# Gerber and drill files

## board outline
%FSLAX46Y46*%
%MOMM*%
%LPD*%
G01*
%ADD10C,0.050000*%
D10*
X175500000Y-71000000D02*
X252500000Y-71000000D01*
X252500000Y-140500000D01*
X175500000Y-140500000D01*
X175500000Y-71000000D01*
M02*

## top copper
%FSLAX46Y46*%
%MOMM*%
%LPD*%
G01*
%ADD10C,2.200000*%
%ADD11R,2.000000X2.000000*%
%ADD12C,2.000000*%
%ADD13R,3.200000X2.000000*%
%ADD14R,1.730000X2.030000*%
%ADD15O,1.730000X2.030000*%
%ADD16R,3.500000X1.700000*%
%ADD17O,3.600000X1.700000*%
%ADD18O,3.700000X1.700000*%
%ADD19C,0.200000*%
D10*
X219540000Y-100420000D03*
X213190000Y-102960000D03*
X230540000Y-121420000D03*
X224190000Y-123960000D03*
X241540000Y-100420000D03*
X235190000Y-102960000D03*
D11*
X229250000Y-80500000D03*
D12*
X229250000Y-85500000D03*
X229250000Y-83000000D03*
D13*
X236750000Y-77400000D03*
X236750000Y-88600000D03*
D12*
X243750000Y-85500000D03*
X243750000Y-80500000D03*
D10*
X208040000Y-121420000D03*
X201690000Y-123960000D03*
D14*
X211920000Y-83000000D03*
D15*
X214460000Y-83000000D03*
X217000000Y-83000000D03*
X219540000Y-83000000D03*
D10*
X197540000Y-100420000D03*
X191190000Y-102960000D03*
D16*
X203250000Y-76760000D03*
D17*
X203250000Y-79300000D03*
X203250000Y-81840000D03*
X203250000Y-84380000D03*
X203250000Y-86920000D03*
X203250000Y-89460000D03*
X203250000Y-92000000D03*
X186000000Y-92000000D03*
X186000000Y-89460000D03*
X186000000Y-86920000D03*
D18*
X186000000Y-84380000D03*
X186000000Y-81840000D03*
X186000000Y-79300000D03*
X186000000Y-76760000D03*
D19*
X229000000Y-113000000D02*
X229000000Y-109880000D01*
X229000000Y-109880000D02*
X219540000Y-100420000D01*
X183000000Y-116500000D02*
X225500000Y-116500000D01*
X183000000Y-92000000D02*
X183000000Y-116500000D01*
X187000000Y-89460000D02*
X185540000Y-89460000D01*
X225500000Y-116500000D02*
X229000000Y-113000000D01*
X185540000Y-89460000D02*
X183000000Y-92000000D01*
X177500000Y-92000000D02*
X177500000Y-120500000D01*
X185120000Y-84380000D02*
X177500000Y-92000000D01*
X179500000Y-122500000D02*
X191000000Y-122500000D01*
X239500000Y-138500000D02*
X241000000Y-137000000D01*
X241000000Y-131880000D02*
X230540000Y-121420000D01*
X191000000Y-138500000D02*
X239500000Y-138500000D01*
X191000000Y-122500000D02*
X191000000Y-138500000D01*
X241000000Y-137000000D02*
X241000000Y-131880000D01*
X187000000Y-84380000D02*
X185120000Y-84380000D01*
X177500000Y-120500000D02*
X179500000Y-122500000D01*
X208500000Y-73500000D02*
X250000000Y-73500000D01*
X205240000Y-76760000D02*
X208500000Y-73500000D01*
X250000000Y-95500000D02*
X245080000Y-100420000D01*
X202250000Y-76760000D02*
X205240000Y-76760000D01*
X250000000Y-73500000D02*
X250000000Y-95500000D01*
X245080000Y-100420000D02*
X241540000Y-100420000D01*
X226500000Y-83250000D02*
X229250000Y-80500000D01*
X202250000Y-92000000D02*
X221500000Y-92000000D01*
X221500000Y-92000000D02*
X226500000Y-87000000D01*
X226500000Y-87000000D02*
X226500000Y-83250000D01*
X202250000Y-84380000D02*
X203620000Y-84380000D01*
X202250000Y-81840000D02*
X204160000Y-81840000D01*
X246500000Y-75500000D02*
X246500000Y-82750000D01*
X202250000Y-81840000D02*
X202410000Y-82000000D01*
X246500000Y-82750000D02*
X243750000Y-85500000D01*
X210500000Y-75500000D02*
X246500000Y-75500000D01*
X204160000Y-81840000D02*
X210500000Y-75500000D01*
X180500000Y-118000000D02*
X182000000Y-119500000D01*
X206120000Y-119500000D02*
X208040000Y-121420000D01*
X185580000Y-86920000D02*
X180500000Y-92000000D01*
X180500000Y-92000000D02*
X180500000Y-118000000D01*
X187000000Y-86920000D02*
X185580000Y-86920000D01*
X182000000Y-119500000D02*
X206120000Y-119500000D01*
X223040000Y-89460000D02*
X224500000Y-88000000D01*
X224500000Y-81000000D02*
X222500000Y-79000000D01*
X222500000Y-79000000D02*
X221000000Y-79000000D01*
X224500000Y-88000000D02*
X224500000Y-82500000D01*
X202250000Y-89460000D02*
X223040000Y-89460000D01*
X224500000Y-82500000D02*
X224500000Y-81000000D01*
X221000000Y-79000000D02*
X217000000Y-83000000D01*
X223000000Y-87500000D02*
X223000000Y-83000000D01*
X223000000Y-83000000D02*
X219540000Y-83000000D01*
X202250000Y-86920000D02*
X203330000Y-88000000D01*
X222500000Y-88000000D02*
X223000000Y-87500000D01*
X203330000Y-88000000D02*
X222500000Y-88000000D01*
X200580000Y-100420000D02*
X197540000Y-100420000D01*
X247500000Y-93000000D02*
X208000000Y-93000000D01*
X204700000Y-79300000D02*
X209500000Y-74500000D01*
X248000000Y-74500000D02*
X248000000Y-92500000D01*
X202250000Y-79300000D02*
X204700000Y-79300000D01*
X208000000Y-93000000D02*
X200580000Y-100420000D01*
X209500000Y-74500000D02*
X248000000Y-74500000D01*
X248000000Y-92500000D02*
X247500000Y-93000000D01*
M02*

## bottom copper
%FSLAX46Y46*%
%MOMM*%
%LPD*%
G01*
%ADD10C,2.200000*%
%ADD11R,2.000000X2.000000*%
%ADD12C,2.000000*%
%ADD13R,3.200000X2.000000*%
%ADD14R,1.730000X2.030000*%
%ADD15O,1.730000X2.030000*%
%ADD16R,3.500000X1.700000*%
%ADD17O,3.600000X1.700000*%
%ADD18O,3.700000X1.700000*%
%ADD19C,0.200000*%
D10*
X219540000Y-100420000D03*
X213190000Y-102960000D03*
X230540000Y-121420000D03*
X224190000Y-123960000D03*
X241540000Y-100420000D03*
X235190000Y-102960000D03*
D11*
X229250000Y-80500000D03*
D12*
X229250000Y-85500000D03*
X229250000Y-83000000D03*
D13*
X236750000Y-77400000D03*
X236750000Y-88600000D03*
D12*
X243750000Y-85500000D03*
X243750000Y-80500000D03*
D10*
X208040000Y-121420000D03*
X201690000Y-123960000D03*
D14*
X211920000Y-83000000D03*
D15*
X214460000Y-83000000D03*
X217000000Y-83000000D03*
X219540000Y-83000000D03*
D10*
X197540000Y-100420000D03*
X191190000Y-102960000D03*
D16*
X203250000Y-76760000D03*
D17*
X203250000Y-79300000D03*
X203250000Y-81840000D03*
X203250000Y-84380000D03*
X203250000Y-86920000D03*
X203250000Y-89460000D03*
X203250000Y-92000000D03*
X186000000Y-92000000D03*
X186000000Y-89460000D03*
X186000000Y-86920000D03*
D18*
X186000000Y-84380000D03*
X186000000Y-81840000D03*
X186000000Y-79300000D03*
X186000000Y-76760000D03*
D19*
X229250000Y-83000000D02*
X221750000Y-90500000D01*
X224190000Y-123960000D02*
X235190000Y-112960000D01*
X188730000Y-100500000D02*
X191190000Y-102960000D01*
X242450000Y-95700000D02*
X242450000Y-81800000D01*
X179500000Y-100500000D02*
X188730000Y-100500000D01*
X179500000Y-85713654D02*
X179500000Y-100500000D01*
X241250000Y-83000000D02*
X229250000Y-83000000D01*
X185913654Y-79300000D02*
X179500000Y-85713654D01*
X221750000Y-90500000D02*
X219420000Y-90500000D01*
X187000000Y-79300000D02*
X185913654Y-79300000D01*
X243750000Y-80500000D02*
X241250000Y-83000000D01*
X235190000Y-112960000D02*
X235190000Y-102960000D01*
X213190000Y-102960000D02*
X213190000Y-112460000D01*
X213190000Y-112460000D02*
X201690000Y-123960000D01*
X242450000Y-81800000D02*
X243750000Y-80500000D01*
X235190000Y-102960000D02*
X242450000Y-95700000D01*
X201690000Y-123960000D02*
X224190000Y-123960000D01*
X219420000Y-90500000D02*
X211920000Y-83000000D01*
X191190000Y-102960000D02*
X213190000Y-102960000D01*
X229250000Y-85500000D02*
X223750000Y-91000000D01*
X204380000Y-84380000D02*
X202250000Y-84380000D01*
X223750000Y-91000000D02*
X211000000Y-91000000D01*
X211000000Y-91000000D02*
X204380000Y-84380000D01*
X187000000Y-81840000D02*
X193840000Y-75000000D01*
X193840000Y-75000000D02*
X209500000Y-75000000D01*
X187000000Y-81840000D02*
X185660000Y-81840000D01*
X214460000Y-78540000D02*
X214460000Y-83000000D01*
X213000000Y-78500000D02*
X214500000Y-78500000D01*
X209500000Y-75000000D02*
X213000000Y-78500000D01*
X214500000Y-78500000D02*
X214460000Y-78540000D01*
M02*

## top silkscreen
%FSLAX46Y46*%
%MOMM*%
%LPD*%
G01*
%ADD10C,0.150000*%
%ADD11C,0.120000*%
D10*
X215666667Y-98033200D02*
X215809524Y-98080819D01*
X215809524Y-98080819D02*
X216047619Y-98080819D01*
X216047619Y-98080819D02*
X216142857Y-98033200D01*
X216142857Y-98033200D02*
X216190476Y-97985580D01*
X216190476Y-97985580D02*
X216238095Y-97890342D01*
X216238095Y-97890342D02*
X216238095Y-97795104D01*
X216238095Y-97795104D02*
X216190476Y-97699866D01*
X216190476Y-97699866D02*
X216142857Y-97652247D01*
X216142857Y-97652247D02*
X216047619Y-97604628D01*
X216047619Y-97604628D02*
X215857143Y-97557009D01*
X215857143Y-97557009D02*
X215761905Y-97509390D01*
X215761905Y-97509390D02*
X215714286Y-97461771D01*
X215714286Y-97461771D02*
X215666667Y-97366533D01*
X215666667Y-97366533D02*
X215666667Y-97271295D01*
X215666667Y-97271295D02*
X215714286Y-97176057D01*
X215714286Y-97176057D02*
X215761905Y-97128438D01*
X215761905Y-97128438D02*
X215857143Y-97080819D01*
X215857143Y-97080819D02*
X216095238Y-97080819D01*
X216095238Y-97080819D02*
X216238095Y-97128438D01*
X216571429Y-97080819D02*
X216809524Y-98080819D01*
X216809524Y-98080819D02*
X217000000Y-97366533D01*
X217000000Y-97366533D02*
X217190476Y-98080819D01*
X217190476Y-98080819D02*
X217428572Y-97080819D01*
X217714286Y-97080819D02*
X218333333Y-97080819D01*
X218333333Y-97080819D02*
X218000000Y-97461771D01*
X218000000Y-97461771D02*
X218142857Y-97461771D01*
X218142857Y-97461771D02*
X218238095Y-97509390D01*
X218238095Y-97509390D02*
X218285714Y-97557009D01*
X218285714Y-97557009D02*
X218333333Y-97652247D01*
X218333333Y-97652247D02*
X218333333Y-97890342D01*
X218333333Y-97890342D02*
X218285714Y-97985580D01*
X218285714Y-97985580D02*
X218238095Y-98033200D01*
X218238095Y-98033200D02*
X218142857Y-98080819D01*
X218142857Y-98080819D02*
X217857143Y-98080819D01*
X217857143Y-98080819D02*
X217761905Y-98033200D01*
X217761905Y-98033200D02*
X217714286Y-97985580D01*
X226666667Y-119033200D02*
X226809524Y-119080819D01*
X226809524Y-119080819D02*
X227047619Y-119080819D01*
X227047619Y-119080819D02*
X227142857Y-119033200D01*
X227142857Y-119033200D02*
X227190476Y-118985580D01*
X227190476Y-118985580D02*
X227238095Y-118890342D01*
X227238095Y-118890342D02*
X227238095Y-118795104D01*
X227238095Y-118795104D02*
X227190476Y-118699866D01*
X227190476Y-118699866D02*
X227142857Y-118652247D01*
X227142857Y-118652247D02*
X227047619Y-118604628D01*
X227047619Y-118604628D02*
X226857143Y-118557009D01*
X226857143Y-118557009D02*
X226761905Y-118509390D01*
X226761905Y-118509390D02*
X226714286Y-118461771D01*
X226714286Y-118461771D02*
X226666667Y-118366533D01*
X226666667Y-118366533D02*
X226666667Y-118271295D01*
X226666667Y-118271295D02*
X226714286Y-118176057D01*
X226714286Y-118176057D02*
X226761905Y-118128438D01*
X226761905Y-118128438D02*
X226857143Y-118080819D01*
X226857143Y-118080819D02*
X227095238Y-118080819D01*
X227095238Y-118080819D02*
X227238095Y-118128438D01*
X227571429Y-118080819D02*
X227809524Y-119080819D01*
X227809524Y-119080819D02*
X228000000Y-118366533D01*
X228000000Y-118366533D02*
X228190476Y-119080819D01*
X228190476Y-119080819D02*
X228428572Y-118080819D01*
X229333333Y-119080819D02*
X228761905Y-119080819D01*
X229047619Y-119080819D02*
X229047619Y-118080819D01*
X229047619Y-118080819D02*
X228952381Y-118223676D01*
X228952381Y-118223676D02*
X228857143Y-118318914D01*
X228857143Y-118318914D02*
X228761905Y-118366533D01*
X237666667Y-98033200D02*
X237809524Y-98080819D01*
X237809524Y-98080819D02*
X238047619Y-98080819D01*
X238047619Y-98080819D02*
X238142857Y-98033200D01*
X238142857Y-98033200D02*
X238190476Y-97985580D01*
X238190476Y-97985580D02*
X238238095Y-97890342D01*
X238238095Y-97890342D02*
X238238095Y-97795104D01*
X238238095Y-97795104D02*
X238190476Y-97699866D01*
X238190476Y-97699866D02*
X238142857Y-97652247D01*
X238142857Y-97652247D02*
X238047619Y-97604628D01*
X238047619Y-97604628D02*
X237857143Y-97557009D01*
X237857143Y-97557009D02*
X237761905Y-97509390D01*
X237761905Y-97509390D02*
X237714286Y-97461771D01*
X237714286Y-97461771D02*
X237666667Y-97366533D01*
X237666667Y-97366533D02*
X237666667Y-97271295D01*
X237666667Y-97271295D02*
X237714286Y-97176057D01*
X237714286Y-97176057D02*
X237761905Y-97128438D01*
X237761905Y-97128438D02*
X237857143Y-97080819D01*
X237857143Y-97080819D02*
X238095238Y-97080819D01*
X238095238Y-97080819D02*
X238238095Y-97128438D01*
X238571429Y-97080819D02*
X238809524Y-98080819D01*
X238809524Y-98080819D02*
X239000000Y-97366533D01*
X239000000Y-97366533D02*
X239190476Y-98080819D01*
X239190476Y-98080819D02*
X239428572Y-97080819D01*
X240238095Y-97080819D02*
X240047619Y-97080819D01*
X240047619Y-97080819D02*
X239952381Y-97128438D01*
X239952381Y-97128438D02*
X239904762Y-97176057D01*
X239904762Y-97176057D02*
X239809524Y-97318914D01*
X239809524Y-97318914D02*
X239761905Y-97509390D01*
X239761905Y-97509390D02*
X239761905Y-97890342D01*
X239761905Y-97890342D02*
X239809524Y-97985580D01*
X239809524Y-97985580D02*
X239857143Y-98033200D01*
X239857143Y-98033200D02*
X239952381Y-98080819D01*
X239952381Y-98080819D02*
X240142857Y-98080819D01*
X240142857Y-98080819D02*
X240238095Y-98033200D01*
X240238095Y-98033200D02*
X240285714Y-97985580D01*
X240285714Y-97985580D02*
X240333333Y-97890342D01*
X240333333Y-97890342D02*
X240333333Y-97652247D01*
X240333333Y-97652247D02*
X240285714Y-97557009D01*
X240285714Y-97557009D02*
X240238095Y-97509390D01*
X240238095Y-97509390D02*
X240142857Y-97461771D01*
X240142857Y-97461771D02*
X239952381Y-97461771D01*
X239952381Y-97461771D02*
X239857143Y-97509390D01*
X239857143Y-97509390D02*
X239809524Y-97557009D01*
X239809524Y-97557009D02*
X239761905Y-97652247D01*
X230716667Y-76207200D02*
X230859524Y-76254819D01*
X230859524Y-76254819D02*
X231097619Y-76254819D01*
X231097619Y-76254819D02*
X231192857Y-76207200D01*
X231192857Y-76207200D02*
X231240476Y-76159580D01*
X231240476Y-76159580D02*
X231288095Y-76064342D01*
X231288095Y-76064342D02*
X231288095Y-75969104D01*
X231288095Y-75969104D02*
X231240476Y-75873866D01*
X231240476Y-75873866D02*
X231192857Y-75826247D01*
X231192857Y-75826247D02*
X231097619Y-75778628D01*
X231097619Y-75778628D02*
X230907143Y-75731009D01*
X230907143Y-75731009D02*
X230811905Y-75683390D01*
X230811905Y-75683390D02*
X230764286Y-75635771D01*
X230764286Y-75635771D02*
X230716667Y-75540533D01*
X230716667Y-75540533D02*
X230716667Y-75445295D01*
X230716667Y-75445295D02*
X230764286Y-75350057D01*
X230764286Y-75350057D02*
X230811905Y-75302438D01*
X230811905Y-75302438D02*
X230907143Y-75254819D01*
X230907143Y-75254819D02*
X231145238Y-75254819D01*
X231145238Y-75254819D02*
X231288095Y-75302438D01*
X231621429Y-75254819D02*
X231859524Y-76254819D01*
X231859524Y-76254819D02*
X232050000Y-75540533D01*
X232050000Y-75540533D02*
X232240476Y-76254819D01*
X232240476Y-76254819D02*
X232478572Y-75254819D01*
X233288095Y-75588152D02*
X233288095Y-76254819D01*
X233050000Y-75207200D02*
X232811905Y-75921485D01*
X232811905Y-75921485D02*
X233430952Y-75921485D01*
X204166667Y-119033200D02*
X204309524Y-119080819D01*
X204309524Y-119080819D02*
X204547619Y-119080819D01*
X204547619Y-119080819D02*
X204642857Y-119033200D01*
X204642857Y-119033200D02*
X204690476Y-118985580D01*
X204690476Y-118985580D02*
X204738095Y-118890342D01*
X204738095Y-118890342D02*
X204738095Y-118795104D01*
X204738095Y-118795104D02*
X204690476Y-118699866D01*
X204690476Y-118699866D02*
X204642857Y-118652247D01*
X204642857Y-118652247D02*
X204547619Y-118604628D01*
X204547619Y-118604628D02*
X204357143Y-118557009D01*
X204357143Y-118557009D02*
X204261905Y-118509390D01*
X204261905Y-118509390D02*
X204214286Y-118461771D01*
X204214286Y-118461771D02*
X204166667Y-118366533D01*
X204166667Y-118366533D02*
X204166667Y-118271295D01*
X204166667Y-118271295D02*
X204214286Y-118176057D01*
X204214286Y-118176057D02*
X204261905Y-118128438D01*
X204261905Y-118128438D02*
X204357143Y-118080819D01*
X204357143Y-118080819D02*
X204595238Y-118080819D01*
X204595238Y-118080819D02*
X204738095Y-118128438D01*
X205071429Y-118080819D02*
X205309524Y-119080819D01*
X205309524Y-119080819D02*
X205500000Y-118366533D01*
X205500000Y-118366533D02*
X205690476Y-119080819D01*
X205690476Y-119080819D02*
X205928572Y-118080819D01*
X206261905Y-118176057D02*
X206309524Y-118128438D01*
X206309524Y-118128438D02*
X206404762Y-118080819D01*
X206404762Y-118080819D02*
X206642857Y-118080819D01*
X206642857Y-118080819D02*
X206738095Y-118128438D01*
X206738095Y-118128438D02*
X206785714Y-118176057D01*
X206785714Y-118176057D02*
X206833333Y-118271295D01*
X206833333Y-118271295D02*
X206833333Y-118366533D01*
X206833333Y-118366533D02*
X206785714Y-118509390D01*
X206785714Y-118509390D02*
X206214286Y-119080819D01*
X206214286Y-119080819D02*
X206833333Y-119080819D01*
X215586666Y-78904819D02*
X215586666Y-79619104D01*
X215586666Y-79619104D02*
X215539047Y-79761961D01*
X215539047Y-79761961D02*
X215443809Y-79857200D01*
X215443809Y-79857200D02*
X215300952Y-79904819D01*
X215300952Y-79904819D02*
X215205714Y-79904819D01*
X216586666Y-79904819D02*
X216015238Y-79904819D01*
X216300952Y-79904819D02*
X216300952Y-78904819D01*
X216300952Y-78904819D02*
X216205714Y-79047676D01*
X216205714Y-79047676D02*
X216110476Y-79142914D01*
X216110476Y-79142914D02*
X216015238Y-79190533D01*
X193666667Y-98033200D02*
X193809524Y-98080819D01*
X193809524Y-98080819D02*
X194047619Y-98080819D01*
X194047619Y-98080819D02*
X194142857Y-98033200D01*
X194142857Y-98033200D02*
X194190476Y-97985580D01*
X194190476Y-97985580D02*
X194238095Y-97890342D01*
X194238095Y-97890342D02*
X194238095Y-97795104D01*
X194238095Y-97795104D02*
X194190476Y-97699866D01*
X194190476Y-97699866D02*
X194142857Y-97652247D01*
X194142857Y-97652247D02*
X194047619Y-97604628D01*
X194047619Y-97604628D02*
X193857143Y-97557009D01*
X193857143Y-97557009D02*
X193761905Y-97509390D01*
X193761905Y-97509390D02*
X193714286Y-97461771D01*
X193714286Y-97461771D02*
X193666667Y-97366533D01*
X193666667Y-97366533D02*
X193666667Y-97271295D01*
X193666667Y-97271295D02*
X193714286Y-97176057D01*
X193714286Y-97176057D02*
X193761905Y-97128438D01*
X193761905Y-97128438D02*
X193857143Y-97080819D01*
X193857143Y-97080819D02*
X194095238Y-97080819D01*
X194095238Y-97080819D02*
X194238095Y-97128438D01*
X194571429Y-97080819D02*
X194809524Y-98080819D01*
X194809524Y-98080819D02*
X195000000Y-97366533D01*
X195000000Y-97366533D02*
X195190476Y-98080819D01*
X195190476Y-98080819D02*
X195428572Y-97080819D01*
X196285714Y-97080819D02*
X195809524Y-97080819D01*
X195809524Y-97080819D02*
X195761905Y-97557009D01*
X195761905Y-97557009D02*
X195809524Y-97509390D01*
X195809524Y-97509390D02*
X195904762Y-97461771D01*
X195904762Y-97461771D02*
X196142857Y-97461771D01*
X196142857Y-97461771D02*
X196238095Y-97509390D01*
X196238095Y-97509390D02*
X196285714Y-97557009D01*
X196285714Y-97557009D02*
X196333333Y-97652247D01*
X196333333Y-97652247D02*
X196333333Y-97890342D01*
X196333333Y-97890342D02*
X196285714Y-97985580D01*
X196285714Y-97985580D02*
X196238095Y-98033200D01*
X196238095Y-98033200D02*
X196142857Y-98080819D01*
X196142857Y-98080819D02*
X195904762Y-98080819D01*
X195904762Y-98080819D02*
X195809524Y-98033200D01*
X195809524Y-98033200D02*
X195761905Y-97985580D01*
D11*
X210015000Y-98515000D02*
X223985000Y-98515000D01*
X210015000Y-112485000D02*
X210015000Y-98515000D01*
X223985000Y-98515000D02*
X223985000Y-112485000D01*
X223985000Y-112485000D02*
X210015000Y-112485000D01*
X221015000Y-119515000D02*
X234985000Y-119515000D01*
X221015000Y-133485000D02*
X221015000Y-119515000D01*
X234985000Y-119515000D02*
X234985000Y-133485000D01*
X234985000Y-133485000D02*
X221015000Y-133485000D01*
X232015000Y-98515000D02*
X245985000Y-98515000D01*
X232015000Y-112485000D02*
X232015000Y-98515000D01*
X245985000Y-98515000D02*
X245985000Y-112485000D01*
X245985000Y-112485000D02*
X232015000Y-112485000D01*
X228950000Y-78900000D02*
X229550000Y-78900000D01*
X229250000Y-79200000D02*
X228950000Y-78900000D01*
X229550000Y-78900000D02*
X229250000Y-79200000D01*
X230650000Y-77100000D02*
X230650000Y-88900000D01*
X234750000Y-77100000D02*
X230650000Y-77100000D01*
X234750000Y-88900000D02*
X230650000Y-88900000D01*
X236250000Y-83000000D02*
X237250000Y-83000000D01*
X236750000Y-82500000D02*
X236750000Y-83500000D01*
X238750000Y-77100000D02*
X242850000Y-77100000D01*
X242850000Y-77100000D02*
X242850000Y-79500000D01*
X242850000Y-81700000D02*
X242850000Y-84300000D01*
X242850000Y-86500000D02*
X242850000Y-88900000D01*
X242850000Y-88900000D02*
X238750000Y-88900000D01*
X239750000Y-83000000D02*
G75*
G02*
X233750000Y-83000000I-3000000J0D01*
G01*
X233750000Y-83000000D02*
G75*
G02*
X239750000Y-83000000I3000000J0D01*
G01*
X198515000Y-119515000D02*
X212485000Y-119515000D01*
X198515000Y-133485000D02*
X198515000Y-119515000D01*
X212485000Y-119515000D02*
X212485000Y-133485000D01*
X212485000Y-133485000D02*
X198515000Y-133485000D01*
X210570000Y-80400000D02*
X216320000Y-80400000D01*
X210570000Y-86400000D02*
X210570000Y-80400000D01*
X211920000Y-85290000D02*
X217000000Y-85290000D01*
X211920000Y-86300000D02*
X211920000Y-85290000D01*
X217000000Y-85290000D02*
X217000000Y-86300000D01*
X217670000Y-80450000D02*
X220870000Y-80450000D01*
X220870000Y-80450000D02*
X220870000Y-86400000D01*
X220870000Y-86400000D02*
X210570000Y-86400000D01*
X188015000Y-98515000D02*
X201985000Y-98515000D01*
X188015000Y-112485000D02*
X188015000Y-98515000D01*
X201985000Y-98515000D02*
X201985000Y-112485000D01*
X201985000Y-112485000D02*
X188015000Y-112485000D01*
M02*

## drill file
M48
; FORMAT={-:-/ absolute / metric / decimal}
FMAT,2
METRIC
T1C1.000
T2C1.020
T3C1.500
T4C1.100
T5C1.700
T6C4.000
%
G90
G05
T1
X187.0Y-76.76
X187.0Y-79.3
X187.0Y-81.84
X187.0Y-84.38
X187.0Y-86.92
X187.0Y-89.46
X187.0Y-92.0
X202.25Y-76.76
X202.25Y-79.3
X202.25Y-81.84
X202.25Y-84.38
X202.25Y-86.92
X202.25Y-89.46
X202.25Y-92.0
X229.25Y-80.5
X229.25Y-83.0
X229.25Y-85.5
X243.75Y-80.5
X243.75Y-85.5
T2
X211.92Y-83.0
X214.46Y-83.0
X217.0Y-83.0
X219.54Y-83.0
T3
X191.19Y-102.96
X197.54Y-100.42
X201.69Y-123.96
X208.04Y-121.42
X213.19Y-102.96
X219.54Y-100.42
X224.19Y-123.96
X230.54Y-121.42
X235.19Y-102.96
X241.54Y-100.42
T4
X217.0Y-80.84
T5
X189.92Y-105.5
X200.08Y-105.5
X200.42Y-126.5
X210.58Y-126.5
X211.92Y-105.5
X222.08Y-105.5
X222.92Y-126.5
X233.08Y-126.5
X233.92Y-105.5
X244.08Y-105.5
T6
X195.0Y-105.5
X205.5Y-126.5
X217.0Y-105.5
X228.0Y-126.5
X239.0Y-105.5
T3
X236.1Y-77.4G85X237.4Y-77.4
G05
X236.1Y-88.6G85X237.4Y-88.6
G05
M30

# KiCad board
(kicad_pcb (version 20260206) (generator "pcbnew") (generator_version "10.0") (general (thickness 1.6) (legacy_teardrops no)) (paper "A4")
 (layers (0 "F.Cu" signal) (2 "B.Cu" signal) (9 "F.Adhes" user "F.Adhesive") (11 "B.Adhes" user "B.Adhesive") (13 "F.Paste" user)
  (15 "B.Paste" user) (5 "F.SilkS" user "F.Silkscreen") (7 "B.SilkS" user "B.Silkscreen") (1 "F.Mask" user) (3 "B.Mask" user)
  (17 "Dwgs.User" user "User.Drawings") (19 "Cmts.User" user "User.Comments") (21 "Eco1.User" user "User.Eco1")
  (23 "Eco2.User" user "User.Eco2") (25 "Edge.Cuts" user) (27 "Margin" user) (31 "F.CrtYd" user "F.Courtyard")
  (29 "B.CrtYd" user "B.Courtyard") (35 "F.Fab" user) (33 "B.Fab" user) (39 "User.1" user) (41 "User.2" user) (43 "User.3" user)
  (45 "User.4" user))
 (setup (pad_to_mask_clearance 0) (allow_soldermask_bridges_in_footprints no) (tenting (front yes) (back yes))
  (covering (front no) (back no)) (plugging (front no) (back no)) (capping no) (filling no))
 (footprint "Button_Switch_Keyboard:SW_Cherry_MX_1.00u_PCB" (layer "F.Cu") (at 219.54 100.42)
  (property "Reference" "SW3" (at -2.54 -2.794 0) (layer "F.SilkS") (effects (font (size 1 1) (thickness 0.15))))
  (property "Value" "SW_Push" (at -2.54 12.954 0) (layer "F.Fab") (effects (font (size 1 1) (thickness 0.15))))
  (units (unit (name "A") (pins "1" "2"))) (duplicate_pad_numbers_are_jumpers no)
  (fp_line (start -9.525 -1.905) (end 4.445 -1.905) (stroke (width 0.12) (type solid)) (layer "F.SilkS"))
  (fp_line (start -9.525 12.065) (end -9.525 -1.905) (stroke (width 0.12) (type solid)) (layer "F.SilkS"))
  (fp_line (start 4.445 -1.905) (end 4.445 12.065) (stroke (width 0.12) (type solid)) (layer "F.SilkS"))
  (fp_line (start 4.445 12.065) (end -9.525 12.065) (stroke (width 0.12) (type solid)) (layer "F.SilkS"))
  (pad "" np_thru_hole circle (at -7.62 5.08) (size 1.7 1.7) (drill 1.7) (layers "*.Cu" "*.Mask"))
  (pad "" np_thru_hole circle (at -2.54 5.08) (size 4 4) (drill 4) (layers "*.Cu" "*.Mask"))
  (pad "" np_thru_hole circle (at 2.54 5.08) (size 1.7 1.7) (drill 1.7) (layers "*.Cu" "*.Mask"))
  (pad "1" thru_hole circle (at 0 0) (size 2.2 2.2) (drill 1.5) (layers "*.Cu" "*.Mask") (remove_unused_layers no)
   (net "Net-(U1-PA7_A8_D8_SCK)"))
  (pad "2" thru_hole circle (at -6.35 2.54) (size 2.2 2.2) (drill 1.5) (layers "*.Cu" "*.Mask") (remove_unused_layers no) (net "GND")))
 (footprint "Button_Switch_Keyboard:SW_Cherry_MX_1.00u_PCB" (layer "F.Cu") (at 230.54 121.42)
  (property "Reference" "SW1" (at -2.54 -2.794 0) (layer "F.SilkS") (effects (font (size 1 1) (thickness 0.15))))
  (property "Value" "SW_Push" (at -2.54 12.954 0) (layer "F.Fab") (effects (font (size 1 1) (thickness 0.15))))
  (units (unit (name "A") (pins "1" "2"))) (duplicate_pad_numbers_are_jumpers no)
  (fp_line (start -9.525 -1.905) (end 4.445 -1.905) (stroke (width 0.12) (type solid)) (layer "F.SilkS"))
  (fp_line (start -9.525 12.065) (end -9.525 -1.905) (stroke (width 0.12) (type solid)) (layer "F.SilkS"))
  (fp_line (start 4.445 -1.905) (end 4.445 12.065) (stroke (width 0.12) (type solid)) (layer "F.SilkS"))
  (fp_line (start 4.445 12.065) (end -9.525 12.065) (stroke (width 0.12) (type solid)) (layer "F.SilkS"))
  (pad "" np_thru_hole circle (at -7.62 5.08) (size 1.7 1.7) (drill 1.7) (layers "*.Cu" "*.Mask"))
  (pad "" np_thru_hole circle (at -2.54 5.08) (size 4 4) (drill 4) (layers "*.Cu" "*.Mask"))
  (pad "" np_thru_hole circle (at 2.54 5.08) (size 1.7 1.7) (drill 1.7) (layers "*.Cu" "*.Mask"))
  (pad "1" thru_hole circle (at 0 0) (size 2.2 2.2) (drill 1.5) (layers "*.Cu" "*.Mask") (remove_unused_layers no)
   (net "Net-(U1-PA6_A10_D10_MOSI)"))
  (pad "2" thru_hole circle (at -6.35 2.54) (size 2.2 2.2) (drill 1.5) (layers "*.Cu" "*.Mask") (remove_unused_layers no) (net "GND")))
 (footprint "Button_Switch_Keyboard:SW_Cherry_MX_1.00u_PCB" (layer "F.Cu") (at 241.54 100.42)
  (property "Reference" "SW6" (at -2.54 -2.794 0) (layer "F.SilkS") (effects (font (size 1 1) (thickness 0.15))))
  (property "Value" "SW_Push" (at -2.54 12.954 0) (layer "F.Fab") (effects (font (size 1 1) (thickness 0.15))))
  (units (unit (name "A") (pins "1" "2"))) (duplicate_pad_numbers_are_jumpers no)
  (fp_line (start -9.525 -1.905) (end 4.445 -1.905) (stroke (width 0.12) (type solid)) (layer "F.SilkS"))
  (fp_line (start -9.525 12.065) (end -9.525 -1.905) (stroke (width 0.12) (type solid)) (layer "F.SilkS"))
  (fp_line (start 4.445 -1.905) (end 4.445 12.065) (stroke (width 0.12) (type solid)) (layer "F.SilkS"))
  (fp_line (start 4.445 12.065) (end -9.525 12.065) (stroke (width 0.12) (type solid)) (layer "F.SilkS"))
  (pad "" np_thru_hole circle (at -7.62 5.08) (size 1.7 1.7) (drill 1.7) (layers "*.Cu" "*.Mask"))
  (pad "" np_thru_hole circle (at -2.54 5.08) (size 4 4) (drill 4) (layers "*.Cu" "*.Mask"))
  (pad "" np_thru_hole circle (at 2.54 5.08) (size 1.7 1.7) (drill 1.7) (layers "*.Cu" "*.Mask"))
  (pad "1" thru_hole circle (at 0 0) (size 2.2 2.2) (drill 1.5) (layers "*.Cu" "*.Mask") (remove_unused_layers no)
   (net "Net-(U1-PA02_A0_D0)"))
  (pad "2" thru_hole circle (at -6.35 2.54) (size 2.2 2.2) (drill 1.5) (layers "*.Cu" "*.Mask") (remove_unused_layers no) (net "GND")))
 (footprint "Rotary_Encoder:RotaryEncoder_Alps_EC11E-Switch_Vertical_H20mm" (layer "F.Cu") (at 229.25 80.5)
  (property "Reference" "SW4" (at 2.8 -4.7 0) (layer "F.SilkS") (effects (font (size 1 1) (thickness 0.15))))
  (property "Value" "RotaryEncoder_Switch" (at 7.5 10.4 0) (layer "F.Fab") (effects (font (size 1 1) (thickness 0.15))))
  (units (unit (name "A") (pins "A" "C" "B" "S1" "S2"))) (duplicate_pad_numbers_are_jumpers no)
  (fp_line (start -0.3 -1.6) (end 0.3 -1.6) (stroke (width 0.12) (type solid)) (layer "F.SilkS"))
  (fp_line (start 0 -1.3) (end -0.3 -1.6) (stroke (width 0.12) (type solid)) (layer "F.SilkS"))
  (fp_line (start 0.3 -1.6) (end 0 -1.3) (stroke (width 0.12) (type solid)) (layer "F.SilkS"))
  (fp_line (start 1.4 -3.4) (end 1.4 8.4) (stroke (width 0.12) (type solid)) (layer "F.SilkS"))
  (fp_line (start 5.5 -3.4) (end 1.4 -3.4) (stroke (width 0.12) (type solid)) (layer "F.SilkS"))
  (fp_line (start 5.5 8.4) (end 1.4 8.4) (stroke (width 0.12) (type solid)) (layer "F.SilkS"))
  (fp_line (start 7 2.5) (end 8 2.5) (stroke (width 0.12) (type solid)) (layer "F.SilkS"))
  (fp_line (start 7.5 2) (end 7.5 3) (stroke (width 0.12) (type solid)) (layer "F.SilkS"))
  (fp_line (start 9.5 -3.4) (end 13.6 -3.4) (stroke (width 0.12) (type solid)) (layer "F.SilkS"))
  (fp_line (start 13.6 -3.4) (end 13.6 -1) (stroke (width 0.12) (type solid)) (layer "F.SilkS"))
  (fp_line (start 13.6 1.2) (end 13.6 3.8) (stroke (width 0.12) (type solid)) (layer "F.SilkS"))
  (fp_line (start 13.6 6) (end 13.6 8.4) (stroke (width 0.12) (type solid)) (layer "F.SilkS"))
  (fp_line (start 13.6 8.4) (end 9.5 8.4) (stroke (width 0.12) (type solid)) (layer "F.SilkS"))
  (fp_circle (center 7.5 2.5) (end 10.5 2.5) (stroke (width 0.12) (type solid)) (fill no) (layer "F.SilkS"))
  (pad "A" thru_hole rect (at 0 0) (size 2 2) (drill 1) (layers "*.Cu" "*.Mask") (remove_unused_layers no) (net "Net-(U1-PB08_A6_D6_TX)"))
  (pad "B" thru_hole circle (at 0 5) (size 2 2) (drill 1) (layers "*.Cu" "*.Mask") (remove_unused_layers no) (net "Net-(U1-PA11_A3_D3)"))
  (pad "C" thru_hole circle (at 0 2.5) (size 2 2) (drill 1) (layers "*.Cu" "*.Mask") (remove_unused_layers no) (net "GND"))
  (pad "MP" thru_hole rect (at 7.5 -3.1) (size 3.2 2) (drill oval 2.8 1.5) (layers "*.Cu" "*.Mask") (remove_unused_layers no))
  (pad "MP" thru_hole rect (at 7.5 8.1) (size 3.2 2) (drill oval 2.8 1.5) (layers "*.Cu" "*.Mask") (remove_unused_layers no))
  (pad "S1" thru_hole circle (at 14.5 5) (size 2 2) (drill 1) (layers "*.Cu" "*.Mask") (remove_unused_layers no) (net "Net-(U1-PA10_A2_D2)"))
  (pad "S2" thru_hole circle (at 14.5 0) (size 2 2) (drill 1) (layers "*.Cu" "*.Mask") (remove_unused_layers no) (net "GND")))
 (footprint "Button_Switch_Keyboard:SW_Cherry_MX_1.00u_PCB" (layer "F.Cu") (at 208.04 121.42)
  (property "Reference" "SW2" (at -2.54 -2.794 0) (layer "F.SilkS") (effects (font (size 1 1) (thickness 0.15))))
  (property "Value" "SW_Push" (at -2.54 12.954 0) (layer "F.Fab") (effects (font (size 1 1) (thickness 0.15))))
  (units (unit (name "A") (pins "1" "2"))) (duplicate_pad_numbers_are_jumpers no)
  (fp_line (start -9.525 -1.905) (end 4.445 -1.905) (stroke (width 0.12) (type solid)) (layer "F.SilkS"))
  (fp_line (start -9.525 12.065) (end -9.525 -1.905) (stroke (width 0.12) (type solid)) (layer "F.SilkS"))
  (fp_line (start 4.445 -1.905) (end 4.445 12.065) (stroke (width 0.12) (type solid)) (layer "F.SilkS"))
  (fp_line (start 4.445 12.065) (end -9.525 12.065) (stroke (width 0.12) (type solid)) (layer "F.SilkS"))
  (pad "" np_thru_hole circle (at -7.62 5.08) (size 1.7 1.7) (drill 1.7) (layers "*.Cu" "*.Mask"))
  (pad "" np_thru_hole circle (at -2.54 5.08) (size 4 4) (drill 4) (layers "*.Cu" "*.Mask"))
  (pad "" np_thru_hole circle (at 2.54 5.08) (size 1.7 1.7) (drill 1.7) (layers "*.Cu" "*.Mask"))
  (pad "1" thru_hole circle (at 0 0) (size 2.2 2.2) (drill 1.5) (layers "*.Cu" "*.Mask") (remove_unused_layers no)
   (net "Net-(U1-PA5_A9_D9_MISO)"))
  (pad "2" thru_hole circle (at -6.35 2.54) (size 2.2 2.2) (drill 1.5) (layers "*.Cu" "*.Mask") (remove_unused_layers no) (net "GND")))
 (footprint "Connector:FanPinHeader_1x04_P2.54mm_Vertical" (layer "F.Cu") (at 211.92 83)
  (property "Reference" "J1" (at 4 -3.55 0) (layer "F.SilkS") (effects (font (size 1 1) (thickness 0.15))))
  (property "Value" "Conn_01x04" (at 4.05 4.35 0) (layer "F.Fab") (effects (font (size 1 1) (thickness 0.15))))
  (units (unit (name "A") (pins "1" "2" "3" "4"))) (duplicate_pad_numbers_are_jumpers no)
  (fp_line (start -1.35 -2.6) (end 4.4 -2.6) (stroke (width 0.12) (type solid)) (layer "F.SilkS"))
  (fp_line (start -1.35 3.4) (end -1.35 -2.6) (stroke (width 0.12) (type solid)) (layer "F.SilkS"))
  (fp_line (start 0 2.29) (end 5.08 2.29) (stroke (width 0.12) (type solid)) (layer "F.SilkS"))
  (fp_line (start 0 3.3) (end 0 2.29) (stroke (width 0.12) (type solid)) (layer "F.SilkS"))
  (fp_line (start 5.08 2.29) (end 5.08 3.3) (stroke (width 0.12) (type solid)) (layer "F.SilkS"))
  (fp_line (start 5.75 -2.55) (end 8.95 -2.55) (stroke (width 0.12) (type solid)) (layer "F.SilkS"))
  (fp_line (start 8.95 -2.55) (end 8.95 3.4) (stroke (width 0.12) (type solid)) (layer "F.SilkS"))
  (fp_line (start 8.95 3.4) (end -1.35 3.4) (stroke (width 0.12) (type solid)) (layer "F.SilkS"))
  (pad "" np_thru_hole circle (at 5.08 -2.16 90) (size 1.1 1.1) (drill 1.1) (layers "*.Cu" "*.Mask"))
  (pad "1" thru_hole rect (at 0 0 90) (size 2.03 1.73) (drill 1.02) (layers "*.Cu" "*.Mask") (remove_unused_layers no) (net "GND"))
  (pad "2" thru_hole oval (at 2.54 0 90) (size 2.03 1.73) (drill 1.02) (layers "*.Cu" "*.Mask") (remove_unused_layers no) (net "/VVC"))
  (pad "3" thru_hole oval (at 5.08 0 90) (size 2.03 1.73) (drill 1.02) (layers "*.Cu" "*.Mask") (remove_unused_layers no) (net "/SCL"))
  (pad "4" thru_hole oval (at 7.62 0 90) (size 2.03 1.73) (drill 1.02) (layers "*.Cu" "*.Mask") (remove_unused_layers no) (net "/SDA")))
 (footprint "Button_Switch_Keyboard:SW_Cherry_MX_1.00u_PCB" (layer "F.Cu") (at 197.54 100.42)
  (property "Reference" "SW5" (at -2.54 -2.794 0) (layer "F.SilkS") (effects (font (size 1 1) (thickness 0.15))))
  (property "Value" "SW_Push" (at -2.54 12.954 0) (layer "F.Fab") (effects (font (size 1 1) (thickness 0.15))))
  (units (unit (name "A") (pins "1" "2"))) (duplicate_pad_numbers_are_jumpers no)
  (fp_line (start -9.525 -1.905) (end 4.445 -1.905) (stroke (width 0.12) (type solid)) (layer "F.SilkS"))
  (fp_line (start -9.525 12.065) (end -9.525 -1.905) (stroke (width 0.12) (type solid)) (layer "F.SilkS"))
  (fp_line (start 4.445 -1.905) (end 4.445 12.065) (stroke (width 0.12) (type solid)) (layer "F.SilkS"))
  (fp_line (start 4.445 12.065) (end -9.525 12.065) (stroke (width 0.12) (type solid)) (layer "F.SilkS"))
  (pad "" np_thru_hole circle (at -7.62 5.08) (size 1.7 1.7) (drill 1.7) (layers "*.Cu" "*.Mask"))
  (pad "" np_thru_hole circle (at -2.54 5.08) (size 4 4) (drill 4) (layers "*.Cu" "*.Mask"))
  (pad "" np_thru_hole circle (at 2.54 5.08) (size 1.7 1.7) (drill 1.7) (layers "*.Cu" "*.Mask"))
  (pad "1" thru_hole circle (at 0 0) (size 2.2 2.2) (drill 1.5) (layers "*.Cu" "*.Mask") (remove_unused_layers no)
   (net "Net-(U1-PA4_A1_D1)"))
  (pad "2" thru_hole circle (at -6.35 2.54) (size 2.2 2.2) (drill 1.5) (layers "*.Cu" "*.Mask") (remove_unused_layers no) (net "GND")))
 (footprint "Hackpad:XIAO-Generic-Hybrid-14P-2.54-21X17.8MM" (layer "B.Cu") (at 194.625 84.38 180)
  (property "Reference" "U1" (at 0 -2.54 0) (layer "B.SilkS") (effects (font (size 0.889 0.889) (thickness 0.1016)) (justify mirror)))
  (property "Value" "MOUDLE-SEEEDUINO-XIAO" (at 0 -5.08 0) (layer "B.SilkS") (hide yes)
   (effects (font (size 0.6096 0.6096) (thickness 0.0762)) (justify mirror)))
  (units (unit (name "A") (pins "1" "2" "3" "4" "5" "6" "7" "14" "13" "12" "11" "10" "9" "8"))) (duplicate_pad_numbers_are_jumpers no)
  (pad "1" thru_hole rect (at -7.625 7.62 180) (size 3.5 1.7) (drill 1 (offset -1 0)) (layers "*.Cu" "*.Mask") (remove_unused_layers no)
   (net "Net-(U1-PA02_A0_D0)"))
  (pad "2" thru_hole oval (at -7.625 5.08 180) (size 3.6 1.7) (drill 1 (offset -1 0)) (layers "*.Cu" "*.Mask") (remove_unused_layers no)
   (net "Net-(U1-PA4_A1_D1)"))
  (pad "3" thru_hole oval (at -7.625 2.54 180) (size 3.6 1.7) (drill 1 (offset -1 0)) (layers "*.Cu" "*.Mask") (remove_unused_layers no)
   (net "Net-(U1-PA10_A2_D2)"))
  (pad "4" thru_hole oval (at -7.625 0 180) (size 3.6 1.7) (drill 1 (offset -1 0)) (layers "*.Cu" "*.Mask") (remove_unused_layers no)
   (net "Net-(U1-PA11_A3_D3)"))
  (pad "5" thru_hole oval (at -7.625 -2.54 180) (size 3.6 1.7) (drill 1 (offset -1 0)) (layers "*.Cu" "*.Mask") (remove_unused_layers no)
   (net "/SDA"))
  (pad "6" thru_hole oval (at -7.625 -5.08) (size 3.6 1.7) (drill 1 (offset 1 0)) (layers "*.Cu" "*.Mask") (remove_unused_layers no)
   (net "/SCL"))
  (pad "7" thru_hole oval (at -7.625 -7.62 180) (size 3.6 1.7) (drill 1 (offset -1 0)) (layers "*.Cu" "*.Mask") (remove_unused_layers no)
   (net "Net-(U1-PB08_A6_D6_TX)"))
  (pad "8" thru_hole oval (at 7.625 -7.62 180) (size 3.6 1.7) (drill 1 (offset 1 0)) (layers "*.Cu" "*.Mask") (remove_unused_layers no)
   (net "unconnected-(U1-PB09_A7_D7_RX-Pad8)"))
  (pad "9" thru_hole oval (at 7.625 -5.08 180) (size 3.6 1.7) (drill 1 (offset 1 0)) (layers "*.Cu" "*.Mask") (remove_unused_layers no)
   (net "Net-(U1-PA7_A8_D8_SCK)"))
  (pad "10" thru_hole oval (at 7.625 -2.54 180) (size 3.6 1.7) (drill 1 (offset 1 0)) (layers "*.Cu" "*.Mask") (remove_unused_layers no)
   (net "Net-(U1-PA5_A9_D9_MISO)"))
  (pad "11" thru_hole oval (at 7.625 0 180) (size 3.7 1.7) (drill 1 (offset 1 0)) (layers "*.Cu" "*.Mask") (remove_unused_layers no)
   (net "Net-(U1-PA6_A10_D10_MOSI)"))
  (pad "12" thru_hole oval (at 7.625 2.54 180) (size 3.7 1.7) (drill 1 (offset 1 0)) (layers "*.Cu" "*.Mask") (remove_unused_layers no)
   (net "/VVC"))
  (pad "13" thru_hole oval (at 7.625 5.08 180) (size 3.7 1.7) (drill 1 (offset 1 0)) (layers "*.Cu" "*.Mask") (remove_unused_layers no)
   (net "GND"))
  (pad "14" thru_hole oval (at 7.625 7.62 180) (size 3.7 1.7) (drill 1 (offset 1 0)) (layers "*.Cu" "*.Mask") (remove_unused_layers no)
   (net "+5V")))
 (gr_rect (start 175.5 71) (end 252.5 140.5) (stroke (width 0.05) (type default)) (fill no) (layer "Edge.Cuts"))
 (segment (start 229 113) (end 229 109.88) (width 0.2) (layer "F.Cu") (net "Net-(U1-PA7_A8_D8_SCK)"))
 (segment (start 229 109.88) (end 219.54 100.42) (width 0.2) (layer "F.Cu") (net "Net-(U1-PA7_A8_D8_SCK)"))
 (segment (start 183 116.5) (end 225.5 116.5) (width 0.2) (layer "F.Cu") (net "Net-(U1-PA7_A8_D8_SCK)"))
 (segment (start 183 92) (end 183 116.5) (width 0.2) (layer "F.Cu") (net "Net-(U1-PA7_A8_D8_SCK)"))
 (segment (start 187 89.46) (end 185.54 89.46) (width 0.2) (layer "F.Cu") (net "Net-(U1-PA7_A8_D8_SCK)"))
 (segment (start 225.5 116.5) (end 229 113) (width 0.2) (layer "F.Cu") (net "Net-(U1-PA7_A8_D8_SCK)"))
 (segment (start 185.54 89.46) (end 183 92) (width 0.2) (layer "F.Cu") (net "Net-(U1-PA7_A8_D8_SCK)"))
 (segment (start 229.25 83) (end 221.75 90.5) (width 0.2) (layer "B.Cu") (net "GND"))
 (segment (start 224.19 123.96) (end 235.19 112.96) (width 0.2) (layer "B.Cu") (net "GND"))
 (segment (start 188.73 100.5) (end 191.19 102.96) (width 0.2) (layer "B.Cu") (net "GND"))
 (segment (start 242.45 95.7) (end 242.45 81.8) (width 0.2) (layer "B.Cu") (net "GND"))
 (segment (start 179.5 100.5) (end 188.73 100.5) (width 0.2) (layer "B.Cu") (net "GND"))
 (segment (start 179.5 85.713654) (end 179.5 100.5) (width 0.2) (layer "B.Cu") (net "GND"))
 (segment (start 241.25 83) (end 229.25 83) (width 0.2) (layer "B.Cu") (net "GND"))
 (segment (start 185.913654 79.3) (end 179.5 85.713654) (width 0.2) (layer "B.Cu") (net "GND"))
 (segment (start 221.75 90.5) (end 219.42 90.5) (width 0.2) (layer "B.Cu") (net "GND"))
 (segment (start 187 79.3) (end 185.913654 79.3) (width 0.2) (layer "B.Cu") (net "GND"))
 (segment (start 243.75 80.5) (end 241.25 83) (width 0.2) (layer "B.Cu") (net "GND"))
 (segment (start 235.19 112.96) (end 235.19 102.96) (width 0.2) (layer "B.Cu") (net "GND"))
 (segment (start 213.19 102.96) (end 213.19 112.46) (width 0.2) (layer "B.Cu") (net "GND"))
 (segment (start 213.19 112.46) (end 201.69 123.96) (width 0.2) (layer "B.Cu") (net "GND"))
 (segment (start 242.45 81.8) (end 243.75 80.5) (width 0.2) (layer "B.Cu") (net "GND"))
 (segment (start 235.19 102.96) (end 242.45 95.7) (width 0.2) (layer "B.Cu") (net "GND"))
 (segment (start 201.69 123.96) (end 224.19 123.96) (width 0.2) (layer "B.Cu") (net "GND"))
 (segment (start 219.42 90.5) (end 211.92 83) (width 0.2) (layer "B.Cu") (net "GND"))
 (segment (start 191.19 102.96) (end 213.19 102.96) (width 0.2) (layer "B.Cu") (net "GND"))
 (segment (start 177.5 92) (end 177.5 120.5) (width 0.2) (layer "F.Cu") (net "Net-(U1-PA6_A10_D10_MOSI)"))
 (segment (start 185.12 84.38) (end 177.5 92) (width 0.2) (layer "F.Cu") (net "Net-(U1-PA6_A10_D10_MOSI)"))
 (segment (start 179.5 122.5) (end 191 122.5) (width 0.2) (layer "F.Cu") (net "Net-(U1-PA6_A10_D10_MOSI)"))
 (segment (start 239.5 138.5) (end 241 137) (width 0.2) (layer "F.Cu") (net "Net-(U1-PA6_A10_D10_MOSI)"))
 (segment (start 241 131.88) (end 230.54 121.42) (width 0.2) (layer "F.Cu") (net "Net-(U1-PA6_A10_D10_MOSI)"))
 (segment (start 191 138.5) (end 239.5 138.5) (width 0.2) (layer "F.Cu") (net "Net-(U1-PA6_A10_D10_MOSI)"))
 (segment (start 191 122.5) (end 191 138.5) (width 0.2) (layer "F.Cu") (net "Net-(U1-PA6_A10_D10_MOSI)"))
 (segment (start 241 137) (end 241 131.88) (width 0.2) (layer "F.Cu") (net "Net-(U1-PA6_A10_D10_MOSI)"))
 (segment (start 187 84.38) (end 185.12 84.38) (width 0.2) (layer "F.Cu") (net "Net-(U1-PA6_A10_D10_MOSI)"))
 (segment (start 177.5 120.5) (end 179.5 122.5) (width 0.2) (layer "F.Cu") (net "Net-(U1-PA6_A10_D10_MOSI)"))
 (segment (start 208.5 73.5) (end 250 73.5) (width 0.2) (layer "F.Cu") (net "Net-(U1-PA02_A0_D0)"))
 (segment (start 205.24 76.76) (end 208.5 73.5) (width 0.2) (layer "F.Cu") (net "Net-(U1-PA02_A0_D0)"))
 (segment (start 250 95.5) (end 245.08 100.42) (width 0.2) (layer "F.Cu") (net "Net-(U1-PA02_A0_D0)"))
 (segment (start 202.25 76.76) (end 205.24 76.76) (width 0.2) (layer "F.Cu") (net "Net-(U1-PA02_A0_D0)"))
 (segment (start 250 73.5) (end 250 95.5) (width 0.2) (layer "F.Cu") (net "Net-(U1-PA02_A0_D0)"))
 (segment (start 245.08 100.42) (end 241.54 100.42) (width 0.2) (layer "F.Cu") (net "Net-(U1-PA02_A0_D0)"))
 (segment (start 226.5 83.25) (end 229.25 80.5) (width 0.2) (layer "F.Cu") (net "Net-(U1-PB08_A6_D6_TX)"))
 (segment (start 202.25 92) (end 221.5 92) (width 0.2) (layer "F.Cu") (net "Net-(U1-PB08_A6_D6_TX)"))
 (segment (start 221.5 92) (end 226.5 87) (width 0.2) (layer "F.Cu") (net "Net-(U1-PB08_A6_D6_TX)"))
 (segment (start 226.5 87) (end 226.5 83.25) (width 0.2) (layer "F.Cu") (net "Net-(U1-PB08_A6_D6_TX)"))
 (segment (start 202.25 84.38) (end 203.62 84.38) (width 0.2) (layer "F.Cu") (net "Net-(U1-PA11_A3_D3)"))
 (segment (start 229.25 85.5) (end 223.75 91) (width 0.2) (layer "B.Cu") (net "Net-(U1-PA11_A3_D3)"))
 (segment (start 204.38 84.38) (end 202.25 84.38) (width 0.2) (layer "B.Cu") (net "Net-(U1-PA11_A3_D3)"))
 (segment (start 223.75 91) (end 211 91) (width 0.2) (layer "B.Cu") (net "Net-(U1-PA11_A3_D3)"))
 (segment (start 211 91) (end 204.38 84.38) (width 0.2) (layer "B.Cu") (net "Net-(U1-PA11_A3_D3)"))
 (segment (start 202.25 81.84) (end 204.16 81.84) (width 0.2) (layer "F.Cu") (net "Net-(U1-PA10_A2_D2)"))
 (segment (start 246.5 75.5) (end 246.5 82.75) (width 0.2) (layer "F.Cu") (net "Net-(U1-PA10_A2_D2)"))
 (segment (start 202.25 81.84) (end 202.41 82) (width 0.2) (layer "F.Cu") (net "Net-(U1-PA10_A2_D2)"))
 (segment (start 246.5 82.75) (end 243.75 85.5) (width 0.2) (layer "F.Cu") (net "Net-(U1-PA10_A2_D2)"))
 (segment (start 210.5 75.5) (end 246.5 75.5) (width 0.2) (layer "F.Cu") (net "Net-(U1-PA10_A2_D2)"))
 (segment (start 204.16 81.84) (end 210.5 75.5) (width 0.2) (layer "F.Cu") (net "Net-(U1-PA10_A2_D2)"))
 (segment (start 180.5 118) (end 182 119.5) (width 0.2) (layer "F.Cu") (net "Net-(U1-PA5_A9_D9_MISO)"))
 (segment (start 206.12 119.5) (end 208.04 121.42) (width 0.2) (layer "F.Cu") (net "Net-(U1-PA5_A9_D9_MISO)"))
 (segment (start 185.58 86.92) (end 180.5 92) (width 0.2) (layer "F.Cu") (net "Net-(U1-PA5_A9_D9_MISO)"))
 (segment (start 180.5 92) (end 180.5 118) (width 0.2) (layer "F.Cu") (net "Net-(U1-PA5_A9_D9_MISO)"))
 (segment (start 187 86.92) (end 185.58 86.92) (width 0.2) (layer "F.Cu") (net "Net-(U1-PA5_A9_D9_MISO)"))
 (segment (start 182 119.5) (end 206.12 119.5) (width 0.2) (layer "F.Cu") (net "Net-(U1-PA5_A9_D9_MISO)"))
 (segment (start 187 81.84) (end 193.84 75) (width 0.2) (layer "B.Cu") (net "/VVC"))
 (segment (start 193.84 75) (end 209.5 75) (width 0.2) (layer "B.Cu") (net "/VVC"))
 (segment (start 187 81.84) (end 185.66 81.84) (width 0.2) (layer "B.Cu") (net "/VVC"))
 (segment (start 214.46 78.54) (end 214.46 83) (width 0.2) (layer "B.Cu") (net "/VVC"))
 (segment (start 213 78.5) (end 214.5 78.5) (width 0.2) (layer "B.Cu") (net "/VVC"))
 (segment (start 209.5 75) (end 213 78.5) (width 0.2) (layer "B.Cu") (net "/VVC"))
 (segment (start 214.5 78.5) (end 214.46 78.54) (width 0.2) (layer "B.Cu") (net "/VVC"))
 (segment (start 223.04 89.46) (end 224.5 88) (width 0.2) (layer "F.Cu") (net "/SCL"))
 (segment (start 224.5 81) (end 222.5 79) (width 0.2) (layer "F.Cu") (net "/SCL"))
 (segment (start 222.5 79) (end 221 79) (width 0.2) (layer "F.Cu") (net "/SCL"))
 (segment (start 224.5 88) (end 224.5 82.5) (width 0.2) (layer "F.Cu") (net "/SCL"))
 (segment (start 202.25 89.46) (end 223.04 89.46) (width 0.2) (layer "F.Cu") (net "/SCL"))
 (segment (start 224.5 82.5) (end 224.5 81) (width 0.2) (layer "F.Cu") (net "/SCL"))
 (segment (start 221 79) (end 217 83) (width 0.2) (layer "F.Cu") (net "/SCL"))
 (segment (start 223 87.5) (end 223 83) (width 0.2) (layer "F.Cu") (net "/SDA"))
 (segment (start 223 83) (end 219.54 83) (width 0.2) (layer "F.Cu") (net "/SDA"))
 (segment (start 202.25 86.92) (end 203.33 88) (width 0.2) (layer "F.Cu") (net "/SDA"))
 (segment (start 222.5 88) (end 223 87.5) (width 0.2) (layer "F.Cu") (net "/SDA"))
 (segment (start 203.33 88) (end 222.5 88) (width 0.2) (layer "F.Cu") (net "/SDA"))
 (segment (start 200.58 100.42) (end 197.54 100.42) (width 0.2) (layer "F.Cu") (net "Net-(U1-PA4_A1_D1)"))
 (segment (start 247.5 93) (end 208 93) (width 0.2) (layer "F.Cu") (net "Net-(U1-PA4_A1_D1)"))
 (segment (start 204.7 79.3) (end 209.5 74.5) (width 0.2) (layer "F.Cu") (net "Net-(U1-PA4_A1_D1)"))
 (segment (start 248 74.5) (end 248 92.5) (width 0.2) (layer "F.Cu") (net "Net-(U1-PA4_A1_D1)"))
 (segment (start 202.25 79.3) (end 204.7 79.3) (width 0.2) (layer "F.Cu") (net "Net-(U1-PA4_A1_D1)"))
 (segment (start 208 93) (end 200.58 100.42) (width 0.2) (layer "F.Cu") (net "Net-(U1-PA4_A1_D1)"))
 (segment (start 209.5 74.5) (end 248 74.5) (width 0.2) (layer "F.Cu") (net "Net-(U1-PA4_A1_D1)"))
 (segment (start 248 92.5) (end 247.5 93) (width 0.2) (layer "F.Cu") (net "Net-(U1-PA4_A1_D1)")))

